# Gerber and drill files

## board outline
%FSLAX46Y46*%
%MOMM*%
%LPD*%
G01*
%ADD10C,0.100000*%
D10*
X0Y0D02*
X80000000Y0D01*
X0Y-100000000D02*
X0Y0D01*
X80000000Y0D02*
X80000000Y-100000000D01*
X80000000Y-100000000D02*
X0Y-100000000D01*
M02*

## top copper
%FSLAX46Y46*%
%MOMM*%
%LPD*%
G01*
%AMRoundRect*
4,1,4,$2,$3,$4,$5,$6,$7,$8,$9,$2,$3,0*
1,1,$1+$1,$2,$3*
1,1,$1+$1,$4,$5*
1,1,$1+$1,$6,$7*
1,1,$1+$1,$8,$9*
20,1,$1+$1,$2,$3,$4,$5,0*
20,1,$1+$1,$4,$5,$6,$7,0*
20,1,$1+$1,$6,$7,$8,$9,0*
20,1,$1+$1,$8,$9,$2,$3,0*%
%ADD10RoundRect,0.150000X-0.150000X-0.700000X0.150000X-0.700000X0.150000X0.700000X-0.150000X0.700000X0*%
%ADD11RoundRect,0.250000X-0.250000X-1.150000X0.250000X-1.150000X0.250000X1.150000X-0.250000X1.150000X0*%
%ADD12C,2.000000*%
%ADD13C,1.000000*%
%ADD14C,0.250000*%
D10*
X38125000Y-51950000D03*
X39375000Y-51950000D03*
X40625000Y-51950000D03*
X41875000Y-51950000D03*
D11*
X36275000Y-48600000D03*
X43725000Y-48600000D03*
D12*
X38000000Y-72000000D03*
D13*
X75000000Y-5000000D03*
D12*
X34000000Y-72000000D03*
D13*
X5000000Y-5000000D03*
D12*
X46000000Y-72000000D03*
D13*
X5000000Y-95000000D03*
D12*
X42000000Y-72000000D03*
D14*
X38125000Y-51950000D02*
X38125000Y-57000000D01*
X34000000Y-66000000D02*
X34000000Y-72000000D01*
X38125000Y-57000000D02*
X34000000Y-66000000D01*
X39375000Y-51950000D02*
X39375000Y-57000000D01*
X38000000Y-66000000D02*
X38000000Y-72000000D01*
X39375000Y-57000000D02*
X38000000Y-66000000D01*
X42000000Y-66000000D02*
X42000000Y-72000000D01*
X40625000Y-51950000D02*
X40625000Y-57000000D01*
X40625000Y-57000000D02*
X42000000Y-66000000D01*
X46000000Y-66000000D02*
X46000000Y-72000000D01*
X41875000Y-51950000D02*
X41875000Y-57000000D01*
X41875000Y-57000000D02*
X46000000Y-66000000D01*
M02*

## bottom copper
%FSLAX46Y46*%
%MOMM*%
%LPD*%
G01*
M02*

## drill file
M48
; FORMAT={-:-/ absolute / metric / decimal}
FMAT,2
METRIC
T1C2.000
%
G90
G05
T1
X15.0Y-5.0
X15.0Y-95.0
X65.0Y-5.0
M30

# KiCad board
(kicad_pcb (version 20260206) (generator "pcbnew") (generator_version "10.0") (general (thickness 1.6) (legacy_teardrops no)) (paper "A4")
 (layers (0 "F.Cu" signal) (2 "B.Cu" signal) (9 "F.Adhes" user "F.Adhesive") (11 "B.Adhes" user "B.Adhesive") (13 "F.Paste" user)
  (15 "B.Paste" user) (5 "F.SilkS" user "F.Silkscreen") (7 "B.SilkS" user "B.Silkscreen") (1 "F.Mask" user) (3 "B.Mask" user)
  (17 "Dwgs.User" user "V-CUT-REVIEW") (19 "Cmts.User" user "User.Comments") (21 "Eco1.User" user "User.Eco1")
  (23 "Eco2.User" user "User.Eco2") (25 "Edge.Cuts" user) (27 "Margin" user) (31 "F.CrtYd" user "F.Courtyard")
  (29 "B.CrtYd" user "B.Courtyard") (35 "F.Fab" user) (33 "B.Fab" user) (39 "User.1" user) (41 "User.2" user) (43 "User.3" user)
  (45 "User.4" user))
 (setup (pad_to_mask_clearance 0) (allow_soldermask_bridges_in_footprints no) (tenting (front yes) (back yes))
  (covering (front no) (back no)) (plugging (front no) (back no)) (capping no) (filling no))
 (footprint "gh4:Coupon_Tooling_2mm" (layer "F.Cu") (at 65 5)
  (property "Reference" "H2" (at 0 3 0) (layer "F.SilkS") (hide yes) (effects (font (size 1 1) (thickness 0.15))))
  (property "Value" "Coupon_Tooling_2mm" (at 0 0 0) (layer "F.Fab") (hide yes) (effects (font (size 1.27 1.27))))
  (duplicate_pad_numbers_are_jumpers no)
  (pad "" np_thru_hole circle (at 0 0) (size 2 2) (drill 2) (layers "*.Cu" "*.Mask") (solder_mask_margin 0.05)))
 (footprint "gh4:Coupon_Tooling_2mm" (layer "F.Cu") (at 15 5)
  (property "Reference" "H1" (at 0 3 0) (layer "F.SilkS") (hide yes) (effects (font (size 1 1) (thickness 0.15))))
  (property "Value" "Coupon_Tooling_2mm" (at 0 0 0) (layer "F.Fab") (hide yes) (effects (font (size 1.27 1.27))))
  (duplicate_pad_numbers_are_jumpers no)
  (pad "" np_thru_hole circle (at 0 0) (size 2 2) (drill 2) (layers "*.Cu" "*.Mask") (solder_mask_margin 0.05)))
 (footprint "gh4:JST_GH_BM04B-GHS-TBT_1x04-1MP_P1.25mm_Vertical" (layer "F.Cu") (at 40 50)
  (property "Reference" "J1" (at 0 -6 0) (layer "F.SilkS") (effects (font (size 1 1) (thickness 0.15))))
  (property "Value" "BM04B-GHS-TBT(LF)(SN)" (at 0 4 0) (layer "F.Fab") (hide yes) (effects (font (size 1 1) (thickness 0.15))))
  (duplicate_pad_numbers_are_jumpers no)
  (pad "1" smd roundrect (at -1.875 1.95) (size 0.6 1.7) (layers "F.Cu" "F.Mask" "F.Paste") (roundrect_rratio 0.25) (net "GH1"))
  (pad "2" smd roundrect (at -0.625 1.95) (size 0.6 1.7) (layers "F.Cu" "F.Mask" "F.Paste") (roundrect_rratio 0.25) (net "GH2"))
  (pad "3" smd roundrect (at 0.625 1.95) (size 0.6 1.7) (layers "F.Cu" "F.Mask" "F.Paste") (roundrect_rratio 0.25) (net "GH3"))
  (pad "4" smd roundrect (at 1.875 1.95) (size 0.6 1.7) (layers "F.Cu" "F.Mask" "F.Paste") (roundrect_rratio 0.25) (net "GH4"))
  (pad "MP" smd roundrect (at -3.725 -1.4) (size 1 2.8) (layers "F.Cu" "F.Mask" "F.Paste") (roundrect_rratio 0.25))
  (pad "MP" smd roundrect (at 3.725 -1.4) (size 1 2.8) (layers "F.Cu" "F.Mask" "F.Paste") (roundrect_rratio 0.25)))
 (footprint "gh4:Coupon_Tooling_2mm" (layer "F.Cu") (at 15 95)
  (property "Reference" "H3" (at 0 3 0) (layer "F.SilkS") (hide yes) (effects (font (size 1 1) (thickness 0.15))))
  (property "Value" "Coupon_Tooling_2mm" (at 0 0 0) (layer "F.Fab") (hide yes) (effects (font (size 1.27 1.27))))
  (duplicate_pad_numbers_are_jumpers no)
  (pad "" np_thru_hole circle (at 0 0) (size 2 2) (drill 2) (layers "*.Cu" "*.Mask") (solder_mask_margin 0.05)))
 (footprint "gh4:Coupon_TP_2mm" (layer "F.Cu") (at 38 72)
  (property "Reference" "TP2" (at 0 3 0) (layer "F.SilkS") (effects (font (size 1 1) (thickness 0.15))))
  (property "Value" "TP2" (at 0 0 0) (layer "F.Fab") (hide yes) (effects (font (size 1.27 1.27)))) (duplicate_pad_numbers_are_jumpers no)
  (pad "1" smd circle (at 0 0) (size 2 2) (layers "F.Cu" "F.Mask") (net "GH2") (solder_mask_margin 0.05)))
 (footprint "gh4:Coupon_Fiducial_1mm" (layer "F.Cu") (at 75 5)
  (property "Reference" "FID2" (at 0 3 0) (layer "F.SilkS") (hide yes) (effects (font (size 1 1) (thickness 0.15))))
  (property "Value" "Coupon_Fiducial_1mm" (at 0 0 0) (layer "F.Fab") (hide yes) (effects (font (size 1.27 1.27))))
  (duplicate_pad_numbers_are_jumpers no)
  (pad "" smd circle (at 0 0) (size 1 1) (layers "F.Cu" "F.Mask") (solder_mask_margin 0.5)))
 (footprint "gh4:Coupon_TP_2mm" (layer "F.Cu") (at 34 72)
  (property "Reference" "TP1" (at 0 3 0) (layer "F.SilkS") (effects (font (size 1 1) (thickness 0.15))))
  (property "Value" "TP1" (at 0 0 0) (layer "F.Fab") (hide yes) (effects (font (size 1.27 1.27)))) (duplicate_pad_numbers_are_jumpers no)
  (pad "1" smd circle (at 0 0) (size 2 2) (layers "F.Cu" "F.Mask") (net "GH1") (solder_mask_margin 0.05)))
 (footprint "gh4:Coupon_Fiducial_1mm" (layer "F.Cu") (at 5 5)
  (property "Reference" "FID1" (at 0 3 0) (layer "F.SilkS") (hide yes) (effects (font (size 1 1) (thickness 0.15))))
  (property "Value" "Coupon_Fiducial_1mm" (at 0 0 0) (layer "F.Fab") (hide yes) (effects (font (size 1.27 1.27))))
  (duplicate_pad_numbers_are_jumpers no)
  (pad "" smd circle (at 0 0) (size 1 1) (layers "F.Cu" "F.Mask") (solder_mask_margin 0.5)))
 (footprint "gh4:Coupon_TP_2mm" (layer "F.Cu") (at 46 72)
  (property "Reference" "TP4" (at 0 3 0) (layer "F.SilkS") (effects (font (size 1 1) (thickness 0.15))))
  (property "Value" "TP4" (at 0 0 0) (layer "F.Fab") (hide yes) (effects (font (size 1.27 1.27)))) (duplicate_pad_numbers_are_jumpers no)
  (pad "1" smd circle (at 0 0) (size 2 2) (layers "F.Cu" "F.Mask") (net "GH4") (solder_mask_margin 0.05)))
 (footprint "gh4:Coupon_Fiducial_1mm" (layer "F.Cu") (at 5 95)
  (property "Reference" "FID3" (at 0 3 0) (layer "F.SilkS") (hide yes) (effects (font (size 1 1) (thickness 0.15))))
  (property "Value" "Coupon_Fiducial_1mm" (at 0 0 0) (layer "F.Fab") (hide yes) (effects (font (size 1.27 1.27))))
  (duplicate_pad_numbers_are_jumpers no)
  (pad "" smd circle (at 0 0) (size 1 1) (layers "F.Cu" "F.Mask") (solder_mask_margin 0.5)))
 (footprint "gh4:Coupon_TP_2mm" (layer "F.Cu") (at 42 72)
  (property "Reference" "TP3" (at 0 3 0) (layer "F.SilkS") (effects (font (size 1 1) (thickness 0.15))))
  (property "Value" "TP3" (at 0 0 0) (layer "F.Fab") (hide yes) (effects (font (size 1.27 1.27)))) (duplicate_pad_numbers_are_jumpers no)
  (pad "1" smd circle (at 0 0) (size 2 2) (layers "F.Cu" "F.Mask") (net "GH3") (solder_mask_margin 0.05)))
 (gr_line (start 0 0) (end 80 0) (stroke (width 0.1) (type default)) (layer "Edge.Cuts"))
 (gr_line (start 0 100) (end 0 0) (stroke (width 0.1) (type default)) (layer "Edge.Cuts"))
 (gr_line (start 80 0) (end 80 100) (stroke (width 0.1) (type default)) (layer "Edge.Cuts"))
 (gr_line (start 80 100) (end 0 100) (stroke (width 0.1) (type default)) (layer "Edge.Cuts"))
 (segment (start 38.125 51.95) (end 38.125 57) (width 0.25) (layer "F.Cu") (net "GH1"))
 (segment (start 34 66) (end 34 72) (width 0.25) (layer "F.Cu") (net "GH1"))
 (segment (start 38.125 57) (end 34 66) (width 0.25) (layer "F.Cu") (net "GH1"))
 (segment (start 39.375 51.95) (end 39.375 57) (width 0.25) (layer "F.Cu") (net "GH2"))
 (segment (start 38 66) (end 38 72) (width 0.25) (layer "F.Cu") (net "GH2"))
 (segment (start 39.375 57) (end 38 66) (width 0.25) (layer "F.Cu") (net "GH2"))
 (segment (start 42 66) (end 42 72) (width 0.25) (layer "F.Cu") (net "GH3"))
 (segment (start 40.625 51.95) (end 40.625 57) (width 0.25) (layer "F.Cu") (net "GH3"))
 (segment (start 40.625 57) (end 42 66) (width 0.25) (layer "F.Cu") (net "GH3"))
 (segment (start 46 66) (end 46 72) (width 0.25) (layer "F.Cu") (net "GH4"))
 (segment (start 41.875 51.95) (end 41.875 57) (width 0.25) (layer "F.Cu") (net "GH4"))
 (segment (start 41.875 57) (end 46 66) (width 0.25) (layer "F.Cu") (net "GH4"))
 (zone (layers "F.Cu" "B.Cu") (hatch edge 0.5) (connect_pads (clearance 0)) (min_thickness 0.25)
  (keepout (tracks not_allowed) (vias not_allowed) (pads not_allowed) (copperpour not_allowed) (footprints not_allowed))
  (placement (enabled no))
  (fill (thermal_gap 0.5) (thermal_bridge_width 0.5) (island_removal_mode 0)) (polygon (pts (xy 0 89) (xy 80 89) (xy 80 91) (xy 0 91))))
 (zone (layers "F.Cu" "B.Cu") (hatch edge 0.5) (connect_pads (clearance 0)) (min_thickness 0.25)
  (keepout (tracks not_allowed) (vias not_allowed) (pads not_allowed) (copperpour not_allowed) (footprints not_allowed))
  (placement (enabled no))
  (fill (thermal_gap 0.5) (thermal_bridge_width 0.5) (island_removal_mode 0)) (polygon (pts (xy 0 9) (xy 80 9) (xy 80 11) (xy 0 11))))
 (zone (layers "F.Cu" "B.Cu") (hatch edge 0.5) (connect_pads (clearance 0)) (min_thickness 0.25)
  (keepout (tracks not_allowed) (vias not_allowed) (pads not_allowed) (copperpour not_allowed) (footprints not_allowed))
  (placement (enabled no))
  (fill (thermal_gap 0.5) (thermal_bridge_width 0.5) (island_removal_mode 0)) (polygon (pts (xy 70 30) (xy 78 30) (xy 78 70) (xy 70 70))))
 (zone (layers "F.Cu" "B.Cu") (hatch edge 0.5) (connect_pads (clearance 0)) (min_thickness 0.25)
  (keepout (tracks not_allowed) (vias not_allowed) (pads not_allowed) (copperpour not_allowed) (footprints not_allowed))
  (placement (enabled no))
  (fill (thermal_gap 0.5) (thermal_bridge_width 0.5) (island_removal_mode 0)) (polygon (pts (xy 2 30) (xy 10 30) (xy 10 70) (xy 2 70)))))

